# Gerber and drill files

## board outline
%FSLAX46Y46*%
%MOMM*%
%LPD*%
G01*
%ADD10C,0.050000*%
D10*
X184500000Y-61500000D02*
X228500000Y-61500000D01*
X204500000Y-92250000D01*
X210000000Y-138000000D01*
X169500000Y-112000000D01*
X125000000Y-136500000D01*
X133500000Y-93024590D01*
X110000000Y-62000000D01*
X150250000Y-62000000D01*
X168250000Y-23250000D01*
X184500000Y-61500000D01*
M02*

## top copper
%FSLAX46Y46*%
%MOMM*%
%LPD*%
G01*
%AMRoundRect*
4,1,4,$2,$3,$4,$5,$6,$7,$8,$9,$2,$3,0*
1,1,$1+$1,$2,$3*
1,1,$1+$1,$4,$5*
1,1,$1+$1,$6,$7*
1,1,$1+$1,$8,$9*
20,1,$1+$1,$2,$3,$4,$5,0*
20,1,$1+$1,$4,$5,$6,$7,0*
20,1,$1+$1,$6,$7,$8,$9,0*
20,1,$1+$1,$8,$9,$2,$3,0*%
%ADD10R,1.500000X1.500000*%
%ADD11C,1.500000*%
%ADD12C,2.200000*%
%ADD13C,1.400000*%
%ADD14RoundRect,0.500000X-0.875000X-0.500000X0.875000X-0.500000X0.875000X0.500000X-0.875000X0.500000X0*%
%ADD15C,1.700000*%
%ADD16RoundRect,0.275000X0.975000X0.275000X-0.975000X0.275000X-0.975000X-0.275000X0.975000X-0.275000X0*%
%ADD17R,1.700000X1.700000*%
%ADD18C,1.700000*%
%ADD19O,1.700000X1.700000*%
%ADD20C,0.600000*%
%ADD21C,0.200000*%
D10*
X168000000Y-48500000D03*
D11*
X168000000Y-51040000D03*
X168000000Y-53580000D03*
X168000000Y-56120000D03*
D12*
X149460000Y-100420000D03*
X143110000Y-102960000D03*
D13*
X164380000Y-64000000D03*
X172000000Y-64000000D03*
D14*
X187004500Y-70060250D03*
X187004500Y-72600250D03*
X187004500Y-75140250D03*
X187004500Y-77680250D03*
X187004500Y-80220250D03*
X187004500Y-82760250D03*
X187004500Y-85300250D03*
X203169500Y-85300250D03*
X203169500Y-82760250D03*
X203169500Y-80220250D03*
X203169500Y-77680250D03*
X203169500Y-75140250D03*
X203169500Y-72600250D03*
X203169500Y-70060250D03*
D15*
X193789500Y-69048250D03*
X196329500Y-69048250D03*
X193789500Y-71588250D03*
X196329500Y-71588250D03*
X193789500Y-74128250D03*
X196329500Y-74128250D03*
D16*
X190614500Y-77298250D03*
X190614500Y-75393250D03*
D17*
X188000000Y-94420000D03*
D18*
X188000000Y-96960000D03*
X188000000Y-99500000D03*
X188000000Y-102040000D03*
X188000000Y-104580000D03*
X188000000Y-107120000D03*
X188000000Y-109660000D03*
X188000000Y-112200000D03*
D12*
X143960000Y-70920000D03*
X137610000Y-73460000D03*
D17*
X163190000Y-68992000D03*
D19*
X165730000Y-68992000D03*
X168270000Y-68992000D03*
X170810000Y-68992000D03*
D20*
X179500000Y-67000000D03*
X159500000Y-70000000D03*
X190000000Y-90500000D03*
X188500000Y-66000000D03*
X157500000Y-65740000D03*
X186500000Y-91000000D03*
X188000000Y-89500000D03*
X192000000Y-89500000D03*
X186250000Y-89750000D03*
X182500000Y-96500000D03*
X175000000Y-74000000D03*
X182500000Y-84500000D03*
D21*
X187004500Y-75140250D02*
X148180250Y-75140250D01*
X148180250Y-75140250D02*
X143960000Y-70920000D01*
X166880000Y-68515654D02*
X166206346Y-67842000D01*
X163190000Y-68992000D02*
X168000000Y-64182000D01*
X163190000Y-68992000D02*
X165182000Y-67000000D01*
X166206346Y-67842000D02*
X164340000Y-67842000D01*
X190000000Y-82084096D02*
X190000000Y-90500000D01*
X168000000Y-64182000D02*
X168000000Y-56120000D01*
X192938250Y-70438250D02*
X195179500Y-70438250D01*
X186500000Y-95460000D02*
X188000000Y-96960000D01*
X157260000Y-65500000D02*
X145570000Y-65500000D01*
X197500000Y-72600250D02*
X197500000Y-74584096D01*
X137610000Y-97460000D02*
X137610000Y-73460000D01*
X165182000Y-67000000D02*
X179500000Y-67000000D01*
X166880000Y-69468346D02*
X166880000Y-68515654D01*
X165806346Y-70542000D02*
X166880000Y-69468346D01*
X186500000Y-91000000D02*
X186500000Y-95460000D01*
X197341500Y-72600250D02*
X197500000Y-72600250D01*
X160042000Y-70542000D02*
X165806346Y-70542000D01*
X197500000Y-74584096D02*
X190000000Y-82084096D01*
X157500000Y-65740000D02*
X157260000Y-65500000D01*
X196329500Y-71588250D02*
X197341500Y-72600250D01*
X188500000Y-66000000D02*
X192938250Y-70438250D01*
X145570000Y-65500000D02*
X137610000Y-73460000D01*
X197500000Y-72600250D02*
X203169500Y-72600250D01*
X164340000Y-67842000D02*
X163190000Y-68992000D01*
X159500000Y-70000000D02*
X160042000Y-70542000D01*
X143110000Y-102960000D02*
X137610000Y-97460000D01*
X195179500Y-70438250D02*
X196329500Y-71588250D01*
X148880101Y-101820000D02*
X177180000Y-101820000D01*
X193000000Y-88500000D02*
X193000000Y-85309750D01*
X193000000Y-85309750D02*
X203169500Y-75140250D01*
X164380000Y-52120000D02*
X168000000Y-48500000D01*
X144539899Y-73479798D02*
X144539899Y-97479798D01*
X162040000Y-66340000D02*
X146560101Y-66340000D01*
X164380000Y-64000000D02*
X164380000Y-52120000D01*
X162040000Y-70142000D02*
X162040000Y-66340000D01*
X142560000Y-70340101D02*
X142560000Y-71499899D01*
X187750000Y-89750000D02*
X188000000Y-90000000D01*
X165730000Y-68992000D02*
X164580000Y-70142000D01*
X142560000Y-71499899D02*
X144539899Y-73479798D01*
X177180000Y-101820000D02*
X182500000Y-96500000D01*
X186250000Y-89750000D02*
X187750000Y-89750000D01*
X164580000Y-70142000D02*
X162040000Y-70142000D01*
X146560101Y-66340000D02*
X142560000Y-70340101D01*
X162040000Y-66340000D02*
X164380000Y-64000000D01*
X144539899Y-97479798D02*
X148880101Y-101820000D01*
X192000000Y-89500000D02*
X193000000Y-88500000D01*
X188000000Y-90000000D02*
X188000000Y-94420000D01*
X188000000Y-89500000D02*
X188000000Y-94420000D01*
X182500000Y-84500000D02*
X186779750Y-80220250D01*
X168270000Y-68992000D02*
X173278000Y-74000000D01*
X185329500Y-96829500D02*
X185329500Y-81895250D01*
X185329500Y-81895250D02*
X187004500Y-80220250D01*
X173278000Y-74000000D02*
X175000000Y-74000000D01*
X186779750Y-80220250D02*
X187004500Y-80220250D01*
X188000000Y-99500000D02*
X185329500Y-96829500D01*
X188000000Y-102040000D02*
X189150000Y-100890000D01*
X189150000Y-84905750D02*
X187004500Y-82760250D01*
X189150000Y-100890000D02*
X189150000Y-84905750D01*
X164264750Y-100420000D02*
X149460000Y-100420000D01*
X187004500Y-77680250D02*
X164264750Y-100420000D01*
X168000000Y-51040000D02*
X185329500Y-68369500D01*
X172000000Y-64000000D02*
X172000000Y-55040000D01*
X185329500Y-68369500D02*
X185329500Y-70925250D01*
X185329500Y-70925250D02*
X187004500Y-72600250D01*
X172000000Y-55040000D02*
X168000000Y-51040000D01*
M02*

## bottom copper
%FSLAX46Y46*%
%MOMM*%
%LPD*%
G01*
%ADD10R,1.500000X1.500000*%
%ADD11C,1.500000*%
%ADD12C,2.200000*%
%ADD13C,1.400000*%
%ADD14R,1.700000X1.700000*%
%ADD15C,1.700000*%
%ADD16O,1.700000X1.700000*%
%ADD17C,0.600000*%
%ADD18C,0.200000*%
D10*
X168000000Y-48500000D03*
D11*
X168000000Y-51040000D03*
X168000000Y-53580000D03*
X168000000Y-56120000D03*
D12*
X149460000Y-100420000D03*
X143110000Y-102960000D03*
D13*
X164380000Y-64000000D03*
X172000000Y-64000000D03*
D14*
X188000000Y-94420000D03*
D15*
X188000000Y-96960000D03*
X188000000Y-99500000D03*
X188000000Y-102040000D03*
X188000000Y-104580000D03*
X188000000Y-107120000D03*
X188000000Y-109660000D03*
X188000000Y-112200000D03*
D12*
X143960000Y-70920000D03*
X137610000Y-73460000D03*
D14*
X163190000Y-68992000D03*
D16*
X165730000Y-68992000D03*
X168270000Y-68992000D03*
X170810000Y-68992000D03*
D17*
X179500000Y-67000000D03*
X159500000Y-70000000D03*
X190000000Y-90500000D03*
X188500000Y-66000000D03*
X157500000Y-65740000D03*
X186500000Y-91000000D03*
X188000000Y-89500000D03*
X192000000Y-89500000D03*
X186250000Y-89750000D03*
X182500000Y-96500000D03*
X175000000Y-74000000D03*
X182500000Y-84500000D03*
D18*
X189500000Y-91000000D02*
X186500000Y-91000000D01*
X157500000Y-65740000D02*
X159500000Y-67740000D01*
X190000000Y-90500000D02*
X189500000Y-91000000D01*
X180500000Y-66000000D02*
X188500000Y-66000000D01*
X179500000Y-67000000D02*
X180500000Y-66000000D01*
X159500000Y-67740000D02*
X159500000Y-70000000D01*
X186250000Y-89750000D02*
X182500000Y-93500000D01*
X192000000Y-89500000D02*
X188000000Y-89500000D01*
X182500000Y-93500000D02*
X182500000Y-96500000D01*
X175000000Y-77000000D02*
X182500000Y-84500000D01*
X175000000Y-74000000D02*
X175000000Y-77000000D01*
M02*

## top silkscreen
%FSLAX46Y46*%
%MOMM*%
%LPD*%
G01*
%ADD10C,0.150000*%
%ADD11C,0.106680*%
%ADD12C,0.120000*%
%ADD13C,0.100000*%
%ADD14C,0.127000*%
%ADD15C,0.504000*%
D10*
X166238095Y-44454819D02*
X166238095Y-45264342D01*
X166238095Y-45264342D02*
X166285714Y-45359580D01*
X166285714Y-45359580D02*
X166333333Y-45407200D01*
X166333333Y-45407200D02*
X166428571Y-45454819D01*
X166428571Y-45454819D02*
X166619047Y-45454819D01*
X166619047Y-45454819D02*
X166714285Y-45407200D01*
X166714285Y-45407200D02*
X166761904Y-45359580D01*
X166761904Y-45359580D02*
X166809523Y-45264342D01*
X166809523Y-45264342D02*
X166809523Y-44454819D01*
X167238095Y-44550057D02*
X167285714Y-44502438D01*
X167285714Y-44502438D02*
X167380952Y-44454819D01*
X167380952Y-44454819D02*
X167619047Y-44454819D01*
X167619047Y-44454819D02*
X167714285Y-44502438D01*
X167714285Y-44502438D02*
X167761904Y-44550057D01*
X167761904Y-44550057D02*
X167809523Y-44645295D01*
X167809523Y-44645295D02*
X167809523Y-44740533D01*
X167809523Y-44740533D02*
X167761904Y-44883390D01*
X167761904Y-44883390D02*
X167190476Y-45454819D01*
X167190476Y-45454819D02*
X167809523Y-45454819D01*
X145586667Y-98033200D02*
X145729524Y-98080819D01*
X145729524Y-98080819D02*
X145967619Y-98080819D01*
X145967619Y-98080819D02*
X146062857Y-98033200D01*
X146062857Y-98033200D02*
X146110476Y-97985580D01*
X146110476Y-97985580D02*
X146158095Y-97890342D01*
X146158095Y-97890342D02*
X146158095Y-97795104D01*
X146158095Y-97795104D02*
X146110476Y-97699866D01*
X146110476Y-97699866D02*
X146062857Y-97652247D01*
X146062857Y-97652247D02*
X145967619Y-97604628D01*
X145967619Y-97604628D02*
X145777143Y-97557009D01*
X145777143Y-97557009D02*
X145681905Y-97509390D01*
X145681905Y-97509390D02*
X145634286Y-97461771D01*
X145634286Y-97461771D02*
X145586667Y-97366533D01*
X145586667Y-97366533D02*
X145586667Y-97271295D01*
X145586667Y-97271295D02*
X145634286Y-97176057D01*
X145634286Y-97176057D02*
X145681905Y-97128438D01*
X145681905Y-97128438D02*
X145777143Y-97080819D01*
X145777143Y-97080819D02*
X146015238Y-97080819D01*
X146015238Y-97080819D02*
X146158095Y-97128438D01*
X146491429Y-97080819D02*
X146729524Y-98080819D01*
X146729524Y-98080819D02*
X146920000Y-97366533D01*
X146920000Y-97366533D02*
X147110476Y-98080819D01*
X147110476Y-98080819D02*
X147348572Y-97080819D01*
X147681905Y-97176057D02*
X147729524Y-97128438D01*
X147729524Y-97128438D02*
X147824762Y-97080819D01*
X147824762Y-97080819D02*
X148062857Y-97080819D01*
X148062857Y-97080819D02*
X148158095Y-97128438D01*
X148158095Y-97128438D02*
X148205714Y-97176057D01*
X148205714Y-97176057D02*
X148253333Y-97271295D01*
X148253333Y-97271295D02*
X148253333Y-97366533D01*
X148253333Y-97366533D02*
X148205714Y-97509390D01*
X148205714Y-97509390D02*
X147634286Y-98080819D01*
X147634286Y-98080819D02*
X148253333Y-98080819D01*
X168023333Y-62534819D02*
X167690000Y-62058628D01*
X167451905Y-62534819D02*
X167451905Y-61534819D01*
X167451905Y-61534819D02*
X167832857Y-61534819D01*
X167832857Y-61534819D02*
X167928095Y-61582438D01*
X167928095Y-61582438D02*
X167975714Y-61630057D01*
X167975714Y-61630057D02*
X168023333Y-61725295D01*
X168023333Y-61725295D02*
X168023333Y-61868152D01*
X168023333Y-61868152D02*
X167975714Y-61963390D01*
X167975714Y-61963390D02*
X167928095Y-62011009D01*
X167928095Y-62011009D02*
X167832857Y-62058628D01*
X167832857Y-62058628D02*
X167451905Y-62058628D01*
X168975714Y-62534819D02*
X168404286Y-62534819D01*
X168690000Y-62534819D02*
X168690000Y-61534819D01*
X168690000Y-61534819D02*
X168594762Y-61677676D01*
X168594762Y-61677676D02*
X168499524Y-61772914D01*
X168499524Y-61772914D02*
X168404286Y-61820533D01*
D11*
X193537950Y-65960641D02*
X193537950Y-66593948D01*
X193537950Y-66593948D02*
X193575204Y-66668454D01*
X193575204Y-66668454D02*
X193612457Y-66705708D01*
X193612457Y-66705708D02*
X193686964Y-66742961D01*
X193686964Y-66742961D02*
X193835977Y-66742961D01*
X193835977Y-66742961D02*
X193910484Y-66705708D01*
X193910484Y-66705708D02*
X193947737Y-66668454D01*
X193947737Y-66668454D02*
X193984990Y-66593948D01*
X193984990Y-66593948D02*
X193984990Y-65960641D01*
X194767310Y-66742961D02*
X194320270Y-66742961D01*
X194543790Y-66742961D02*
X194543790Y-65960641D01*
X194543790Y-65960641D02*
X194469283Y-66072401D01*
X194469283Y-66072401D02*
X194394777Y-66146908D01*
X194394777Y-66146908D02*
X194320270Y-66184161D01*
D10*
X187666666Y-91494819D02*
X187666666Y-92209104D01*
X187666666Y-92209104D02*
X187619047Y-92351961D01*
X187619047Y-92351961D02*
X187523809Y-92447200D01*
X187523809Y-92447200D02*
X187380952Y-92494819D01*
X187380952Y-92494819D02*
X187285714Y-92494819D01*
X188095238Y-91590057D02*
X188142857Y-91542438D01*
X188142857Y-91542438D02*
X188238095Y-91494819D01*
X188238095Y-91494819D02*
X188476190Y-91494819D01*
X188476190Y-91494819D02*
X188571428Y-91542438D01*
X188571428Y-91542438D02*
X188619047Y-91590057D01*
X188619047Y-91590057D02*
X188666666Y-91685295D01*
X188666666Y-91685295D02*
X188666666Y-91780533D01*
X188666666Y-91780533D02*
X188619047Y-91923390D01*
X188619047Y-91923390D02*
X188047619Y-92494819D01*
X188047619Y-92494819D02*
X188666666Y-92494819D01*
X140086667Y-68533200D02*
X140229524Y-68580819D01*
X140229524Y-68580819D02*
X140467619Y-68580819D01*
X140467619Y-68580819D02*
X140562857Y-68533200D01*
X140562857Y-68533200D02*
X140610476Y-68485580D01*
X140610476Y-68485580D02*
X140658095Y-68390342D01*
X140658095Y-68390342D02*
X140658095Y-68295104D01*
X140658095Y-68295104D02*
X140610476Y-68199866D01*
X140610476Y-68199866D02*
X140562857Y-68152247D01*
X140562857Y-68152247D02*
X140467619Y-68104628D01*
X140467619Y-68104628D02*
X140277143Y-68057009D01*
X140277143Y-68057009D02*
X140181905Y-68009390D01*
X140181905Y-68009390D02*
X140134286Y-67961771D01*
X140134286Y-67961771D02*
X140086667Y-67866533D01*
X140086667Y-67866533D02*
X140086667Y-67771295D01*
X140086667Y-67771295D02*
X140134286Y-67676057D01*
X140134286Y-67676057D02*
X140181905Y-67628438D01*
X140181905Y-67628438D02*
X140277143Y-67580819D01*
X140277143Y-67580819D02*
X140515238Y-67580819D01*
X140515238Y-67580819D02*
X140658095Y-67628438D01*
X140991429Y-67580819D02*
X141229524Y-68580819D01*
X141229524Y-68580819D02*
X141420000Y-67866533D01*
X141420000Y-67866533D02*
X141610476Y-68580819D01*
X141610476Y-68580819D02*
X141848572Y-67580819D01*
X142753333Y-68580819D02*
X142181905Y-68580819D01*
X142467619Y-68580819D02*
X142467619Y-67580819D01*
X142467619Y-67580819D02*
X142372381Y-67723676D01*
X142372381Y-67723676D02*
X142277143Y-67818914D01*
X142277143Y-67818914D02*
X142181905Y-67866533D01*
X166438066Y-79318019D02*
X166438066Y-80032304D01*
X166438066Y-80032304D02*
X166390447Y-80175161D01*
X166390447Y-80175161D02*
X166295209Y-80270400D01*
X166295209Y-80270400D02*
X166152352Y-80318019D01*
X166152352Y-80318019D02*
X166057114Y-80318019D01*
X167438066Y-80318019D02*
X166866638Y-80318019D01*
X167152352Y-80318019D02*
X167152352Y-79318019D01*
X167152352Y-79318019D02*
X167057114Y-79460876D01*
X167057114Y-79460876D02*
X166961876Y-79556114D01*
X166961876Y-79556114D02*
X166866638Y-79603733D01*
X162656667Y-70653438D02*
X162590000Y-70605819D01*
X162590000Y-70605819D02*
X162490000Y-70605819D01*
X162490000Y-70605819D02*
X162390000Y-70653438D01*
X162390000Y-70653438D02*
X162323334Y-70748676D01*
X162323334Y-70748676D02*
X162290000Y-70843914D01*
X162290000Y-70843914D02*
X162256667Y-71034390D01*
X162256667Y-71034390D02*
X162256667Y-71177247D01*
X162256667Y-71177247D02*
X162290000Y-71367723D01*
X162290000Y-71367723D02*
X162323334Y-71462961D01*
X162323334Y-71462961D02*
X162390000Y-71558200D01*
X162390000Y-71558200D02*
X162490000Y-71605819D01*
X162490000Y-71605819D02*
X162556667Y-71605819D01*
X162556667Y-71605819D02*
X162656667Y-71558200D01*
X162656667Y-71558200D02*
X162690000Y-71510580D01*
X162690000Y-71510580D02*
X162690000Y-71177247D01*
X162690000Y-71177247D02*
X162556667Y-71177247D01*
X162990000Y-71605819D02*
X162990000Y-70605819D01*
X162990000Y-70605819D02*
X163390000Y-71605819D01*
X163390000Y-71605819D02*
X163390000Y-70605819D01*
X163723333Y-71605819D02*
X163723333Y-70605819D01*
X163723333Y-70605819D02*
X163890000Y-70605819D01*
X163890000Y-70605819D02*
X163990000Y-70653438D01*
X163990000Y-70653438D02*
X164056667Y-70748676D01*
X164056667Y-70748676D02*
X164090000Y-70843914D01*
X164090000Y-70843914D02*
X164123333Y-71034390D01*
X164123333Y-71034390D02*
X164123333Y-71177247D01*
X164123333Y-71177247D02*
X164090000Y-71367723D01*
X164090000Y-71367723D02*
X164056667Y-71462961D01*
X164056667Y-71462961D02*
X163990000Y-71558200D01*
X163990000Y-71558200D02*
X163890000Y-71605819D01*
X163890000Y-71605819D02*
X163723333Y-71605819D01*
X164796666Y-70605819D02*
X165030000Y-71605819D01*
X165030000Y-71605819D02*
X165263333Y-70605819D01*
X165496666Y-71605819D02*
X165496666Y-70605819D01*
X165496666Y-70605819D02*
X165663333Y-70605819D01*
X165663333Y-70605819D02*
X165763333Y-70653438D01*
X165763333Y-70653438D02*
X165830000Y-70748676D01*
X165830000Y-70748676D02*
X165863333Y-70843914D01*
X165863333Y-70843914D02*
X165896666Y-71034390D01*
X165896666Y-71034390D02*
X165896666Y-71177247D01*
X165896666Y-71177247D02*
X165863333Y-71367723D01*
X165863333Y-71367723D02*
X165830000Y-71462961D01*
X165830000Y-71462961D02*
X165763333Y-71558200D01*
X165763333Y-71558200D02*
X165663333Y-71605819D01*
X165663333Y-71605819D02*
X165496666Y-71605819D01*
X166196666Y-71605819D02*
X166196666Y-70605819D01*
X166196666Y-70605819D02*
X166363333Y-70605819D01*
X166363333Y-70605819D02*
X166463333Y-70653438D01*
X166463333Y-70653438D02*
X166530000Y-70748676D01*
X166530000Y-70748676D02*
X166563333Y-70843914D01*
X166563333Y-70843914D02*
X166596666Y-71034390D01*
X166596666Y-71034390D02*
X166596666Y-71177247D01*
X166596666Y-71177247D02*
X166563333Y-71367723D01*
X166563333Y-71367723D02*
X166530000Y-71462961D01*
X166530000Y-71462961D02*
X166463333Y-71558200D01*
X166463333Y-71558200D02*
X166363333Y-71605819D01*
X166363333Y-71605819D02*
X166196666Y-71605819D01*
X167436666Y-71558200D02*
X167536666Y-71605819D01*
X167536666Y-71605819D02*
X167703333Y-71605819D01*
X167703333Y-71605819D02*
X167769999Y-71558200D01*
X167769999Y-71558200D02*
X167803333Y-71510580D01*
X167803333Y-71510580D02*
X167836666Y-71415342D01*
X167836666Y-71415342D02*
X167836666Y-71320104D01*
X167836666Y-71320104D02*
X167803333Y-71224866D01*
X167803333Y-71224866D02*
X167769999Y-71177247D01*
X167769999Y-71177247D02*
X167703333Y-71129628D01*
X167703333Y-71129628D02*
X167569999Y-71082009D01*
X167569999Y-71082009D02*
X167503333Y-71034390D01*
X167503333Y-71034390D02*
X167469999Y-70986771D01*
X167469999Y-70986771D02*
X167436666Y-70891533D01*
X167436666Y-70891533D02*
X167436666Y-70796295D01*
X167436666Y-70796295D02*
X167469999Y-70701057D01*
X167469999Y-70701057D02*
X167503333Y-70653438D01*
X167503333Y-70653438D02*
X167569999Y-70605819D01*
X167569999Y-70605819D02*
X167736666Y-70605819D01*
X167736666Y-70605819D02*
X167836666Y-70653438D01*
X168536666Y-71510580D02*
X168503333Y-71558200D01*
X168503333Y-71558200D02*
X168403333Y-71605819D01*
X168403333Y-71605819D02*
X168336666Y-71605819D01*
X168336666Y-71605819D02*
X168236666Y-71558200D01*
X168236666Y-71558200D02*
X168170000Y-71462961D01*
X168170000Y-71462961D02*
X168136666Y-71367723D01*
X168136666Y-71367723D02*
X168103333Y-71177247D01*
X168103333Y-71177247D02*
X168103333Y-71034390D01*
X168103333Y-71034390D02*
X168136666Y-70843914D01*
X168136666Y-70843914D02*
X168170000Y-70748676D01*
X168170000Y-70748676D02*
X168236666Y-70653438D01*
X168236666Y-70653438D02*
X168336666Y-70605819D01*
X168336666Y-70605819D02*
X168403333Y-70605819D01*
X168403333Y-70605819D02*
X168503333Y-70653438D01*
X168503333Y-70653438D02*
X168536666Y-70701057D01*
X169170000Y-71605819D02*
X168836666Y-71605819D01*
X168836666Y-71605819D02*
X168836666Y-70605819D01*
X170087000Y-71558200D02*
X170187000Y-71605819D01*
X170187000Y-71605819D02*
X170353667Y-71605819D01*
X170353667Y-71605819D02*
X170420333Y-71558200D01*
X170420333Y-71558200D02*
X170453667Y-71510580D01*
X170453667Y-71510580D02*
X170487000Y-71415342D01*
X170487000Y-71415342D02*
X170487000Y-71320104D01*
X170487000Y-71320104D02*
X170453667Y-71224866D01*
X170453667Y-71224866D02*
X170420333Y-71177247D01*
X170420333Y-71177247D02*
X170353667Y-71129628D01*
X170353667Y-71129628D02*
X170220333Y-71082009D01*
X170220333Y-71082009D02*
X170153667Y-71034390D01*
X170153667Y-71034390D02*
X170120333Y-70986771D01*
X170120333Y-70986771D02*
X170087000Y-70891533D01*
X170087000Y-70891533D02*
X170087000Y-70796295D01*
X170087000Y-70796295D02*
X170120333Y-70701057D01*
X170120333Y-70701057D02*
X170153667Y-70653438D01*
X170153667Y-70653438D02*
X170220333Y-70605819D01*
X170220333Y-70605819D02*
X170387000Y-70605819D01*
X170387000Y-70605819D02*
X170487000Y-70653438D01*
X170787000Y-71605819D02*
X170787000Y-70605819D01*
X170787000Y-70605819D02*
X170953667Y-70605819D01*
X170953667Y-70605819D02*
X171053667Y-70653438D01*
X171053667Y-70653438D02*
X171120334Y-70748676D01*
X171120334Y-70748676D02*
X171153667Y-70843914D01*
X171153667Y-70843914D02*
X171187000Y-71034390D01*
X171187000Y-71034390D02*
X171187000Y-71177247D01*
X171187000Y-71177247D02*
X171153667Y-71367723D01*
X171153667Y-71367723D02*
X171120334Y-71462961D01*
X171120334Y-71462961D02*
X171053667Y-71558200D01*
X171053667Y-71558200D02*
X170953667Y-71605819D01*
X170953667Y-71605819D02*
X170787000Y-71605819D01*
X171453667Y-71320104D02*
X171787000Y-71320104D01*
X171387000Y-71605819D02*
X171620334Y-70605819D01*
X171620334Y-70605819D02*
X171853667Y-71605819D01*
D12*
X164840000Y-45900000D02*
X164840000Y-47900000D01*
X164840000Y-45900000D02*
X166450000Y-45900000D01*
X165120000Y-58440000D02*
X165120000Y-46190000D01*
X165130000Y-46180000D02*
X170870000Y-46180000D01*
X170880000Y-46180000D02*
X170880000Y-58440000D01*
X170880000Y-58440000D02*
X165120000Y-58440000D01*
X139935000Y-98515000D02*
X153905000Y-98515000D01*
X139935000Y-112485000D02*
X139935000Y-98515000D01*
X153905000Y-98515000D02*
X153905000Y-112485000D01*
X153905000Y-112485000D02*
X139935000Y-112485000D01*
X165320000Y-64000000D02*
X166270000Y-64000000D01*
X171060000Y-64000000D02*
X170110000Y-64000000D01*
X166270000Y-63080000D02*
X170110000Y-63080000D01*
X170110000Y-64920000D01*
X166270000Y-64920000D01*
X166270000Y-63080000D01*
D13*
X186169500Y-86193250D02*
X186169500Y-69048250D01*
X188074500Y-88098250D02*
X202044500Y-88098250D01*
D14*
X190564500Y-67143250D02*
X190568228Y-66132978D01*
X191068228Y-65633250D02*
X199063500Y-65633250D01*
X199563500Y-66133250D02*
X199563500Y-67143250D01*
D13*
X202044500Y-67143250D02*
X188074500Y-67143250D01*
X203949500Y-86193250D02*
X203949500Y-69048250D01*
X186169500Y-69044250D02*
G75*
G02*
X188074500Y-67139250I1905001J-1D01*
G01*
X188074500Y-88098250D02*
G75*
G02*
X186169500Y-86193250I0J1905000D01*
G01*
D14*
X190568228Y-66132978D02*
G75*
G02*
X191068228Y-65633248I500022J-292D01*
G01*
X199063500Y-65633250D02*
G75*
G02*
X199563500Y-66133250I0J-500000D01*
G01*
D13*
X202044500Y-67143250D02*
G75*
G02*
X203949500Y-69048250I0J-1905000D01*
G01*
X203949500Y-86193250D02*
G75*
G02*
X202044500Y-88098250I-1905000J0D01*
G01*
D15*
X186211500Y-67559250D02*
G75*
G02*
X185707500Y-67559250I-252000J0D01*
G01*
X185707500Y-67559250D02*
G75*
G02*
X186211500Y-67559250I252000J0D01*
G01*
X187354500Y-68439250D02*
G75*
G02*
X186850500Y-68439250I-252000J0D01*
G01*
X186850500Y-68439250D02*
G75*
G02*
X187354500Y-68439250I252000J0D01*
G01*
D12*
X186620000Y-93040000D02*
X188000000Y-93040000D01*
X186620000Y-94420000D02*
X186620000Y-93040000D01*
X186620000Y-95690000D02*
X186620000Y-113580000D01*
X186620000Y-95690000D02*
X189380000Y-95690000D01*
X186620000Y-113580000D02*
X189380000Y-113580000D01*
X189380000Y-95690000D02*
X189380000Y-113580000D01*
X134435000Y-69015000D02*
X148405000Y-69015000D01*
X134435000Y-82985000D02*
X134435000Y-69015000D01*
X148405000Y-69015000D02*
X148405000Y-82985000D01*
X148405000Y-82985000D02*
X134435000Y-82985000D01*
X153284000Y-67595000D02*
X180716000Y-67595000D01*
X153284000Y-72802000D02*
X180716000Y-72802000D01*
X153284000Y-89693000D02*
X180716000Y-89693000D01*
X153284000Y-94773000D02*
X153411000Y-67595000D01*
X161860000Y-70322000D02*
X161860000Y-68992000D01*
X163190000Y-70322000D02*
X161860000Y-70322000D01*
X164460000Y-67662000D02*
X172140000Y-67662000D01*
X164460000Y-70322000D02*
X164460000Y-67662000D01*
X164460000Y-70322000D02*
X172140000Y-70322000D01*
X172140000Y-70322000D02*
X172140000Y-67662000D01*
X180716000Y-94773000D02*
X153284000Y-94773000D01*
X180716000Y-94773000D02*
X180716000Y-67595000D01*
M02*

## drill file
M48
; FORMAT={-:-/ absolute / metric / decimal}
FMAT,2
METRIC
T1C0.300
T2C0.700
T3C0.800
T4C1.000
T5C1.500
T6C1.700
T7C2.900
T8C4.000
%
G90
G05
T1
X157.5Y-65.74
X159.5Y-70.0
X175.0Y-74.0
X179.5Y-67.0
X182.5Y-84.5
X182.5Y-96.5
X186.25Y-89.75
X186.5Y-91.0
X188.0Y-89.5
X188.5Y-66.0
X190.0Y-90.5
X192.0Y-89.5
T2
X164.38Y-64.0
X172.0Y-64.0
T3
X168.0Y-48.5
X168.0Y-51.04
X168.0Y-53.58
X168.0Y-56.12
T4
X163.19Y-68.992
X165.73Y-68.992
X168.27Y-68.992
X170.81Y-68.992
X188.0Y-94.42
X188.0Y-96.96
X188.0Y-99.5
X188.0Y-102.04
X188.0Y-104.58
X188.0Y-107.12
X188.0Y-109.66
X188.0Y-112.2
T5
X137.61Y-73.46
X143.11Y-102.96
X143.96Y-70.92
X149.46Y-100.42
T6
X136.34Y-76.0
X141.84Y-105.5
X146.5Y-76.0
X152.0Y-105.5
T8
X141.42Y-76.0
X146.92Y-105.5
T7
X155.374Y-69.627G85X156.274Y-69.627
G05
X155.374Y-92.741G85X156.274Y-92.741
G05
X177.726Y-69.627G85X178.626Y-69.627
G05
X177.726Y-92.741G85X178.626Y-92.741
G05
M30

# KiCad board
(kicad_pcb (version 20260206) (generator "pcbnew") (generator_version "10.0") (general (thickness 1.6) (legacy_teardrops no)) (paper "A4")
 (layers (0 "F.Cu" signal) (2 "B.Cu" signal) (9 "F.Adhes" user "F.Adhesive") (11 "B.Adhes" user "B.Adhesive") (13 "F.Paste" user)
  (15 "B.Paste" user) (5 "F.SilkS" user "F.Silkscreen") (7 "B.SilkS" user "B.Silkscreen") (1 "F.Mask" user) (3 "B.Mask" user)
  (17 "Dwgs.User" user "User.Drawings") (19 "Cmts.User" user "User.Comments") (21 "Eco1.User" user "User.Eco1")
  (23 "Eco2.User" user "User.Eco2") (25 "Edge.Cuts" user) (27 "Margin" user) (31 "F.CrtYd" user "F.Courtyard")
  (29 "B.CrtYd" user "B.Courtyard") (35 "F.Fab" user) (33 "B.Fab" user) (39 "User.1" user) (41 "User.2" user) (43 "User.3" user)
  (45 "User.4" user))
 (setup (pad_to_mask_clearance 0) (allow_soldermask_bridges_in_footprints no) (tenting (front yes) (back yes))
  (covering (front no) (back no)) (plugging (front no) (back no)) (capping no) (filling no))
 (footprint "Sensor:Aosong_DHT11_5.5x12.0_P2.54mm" (layer "F.Cu") (at 168 48.5)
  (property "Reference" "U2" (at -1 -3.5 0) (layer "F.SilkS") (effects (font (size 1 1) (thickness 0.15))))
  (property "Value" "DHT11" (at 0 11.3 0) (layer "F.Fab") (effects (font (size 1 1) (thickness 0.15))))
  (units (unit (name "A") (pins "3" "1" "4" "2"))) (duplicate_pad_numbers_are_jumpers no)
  (fp_line (start -3.16 -2.6) (end -3.16 -0.6) (stroke (width 0.12) (type solid)) (layer "F.SilkS"))
  (fp_line (start -3.16 -2.6) (end -1.55 -2.6) (stroke (width 0.12) (type solid)) (layer "F.SilkS"))
  (fp_line (start -2.88 9.94) (end -2.88 -2.31) (stroke (width 0.12) (type solid)) (layer "F.SilkS"))
  (fp_line (start -2.87 -2.32) (end 2.87 -2.32) (stroke (width 0.12) (type solid)) (layer "F.SilkS"))
  (fp_line (start 2.88 -2.32) (end 2.88 9.94) (stroke (width 0.12) (type solid)) (layer "F.SilkS"))
  (fp_line (start 2.88 9.94) (end -2.88 9.94) (stroke (width 0.12) (type solid)) (layer "F.SilkS"))
  (pad "1" thru_hole rect (at 0 0) (size 1.5 1.5) (drill 0.8) (layers "*.Cu" "*.Mask") (remove_unused_layers no) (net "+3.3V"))
  (pad "2" thru_hole circle (at 0 2.54) (size 1.5 1.5) (drill 0.8) (layers "*.Cu" "*.Mask") (remove_unused_layers no) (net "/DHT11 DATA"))
  (pad "3" thru_hole circle (at 0 5.08) (size 1.5 1.5) (drill 0.8) (layers "*.Cu" "*.Mask") (remove_unused_layers no)
   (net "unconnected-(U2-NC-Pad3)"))
  (pad "4" thru_hole circle (at 0 7.62) (size 1.5 1.5) (drill 0.8) (layers "*.Cu" "*.Mask") (remove_unused_layers no) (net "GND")))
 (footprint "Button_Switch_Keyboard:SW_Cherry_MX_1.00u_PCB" (layer "F.Cu") (at 149.46 100.42)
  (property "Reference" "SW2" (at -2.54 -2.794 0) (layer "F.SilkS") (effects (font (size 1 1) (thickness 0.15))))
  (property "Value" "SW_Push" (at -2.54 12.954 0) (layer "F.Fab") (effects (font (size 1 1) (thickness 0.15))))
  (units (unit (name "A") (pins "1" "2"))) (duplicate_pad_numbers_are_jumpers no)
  (fp_line (start -9.525 -1.905) (end 4.445 -1.905) (stroke (width 0.12) (type solid)) (layer "F.SilkS"))
  (fp_line (start -9.525 12.065) (end -9.525 -1.905) (stroke (width 0.12) (type solid)) (layer "F.SilkS"))
  (fp_line (start 4.445 -1.905) (end 4.445 12.065) (stroke (width 0.12) (type solid)) (layer "F.SilkS"))
  (fp_line (start 4.445 12.065) (end -9.525 12.065) (stroke (width 0.12) (type solid)) (layer "F.SilkS"))
  (pad "" np_thru_hole circle (at -7.62 5.08) (size 1.7 1.7) (drill 1.7) (layers "*.Cu" "*.Mask"))
  (pad "" np_thru_hole circle (at -2.54 5.08) (size 4 4) (drill 4) (layers "*.Cu" "*.Mask"))
  (pad "" np_thru_hole circle (at 2.54 5.08) (size 1.7 1.7) (drill 1.7) (layers "*.Cu" "*.Mask"))
  (pad "1" thru_hole circle (at 0 0) (size 2.2 2.2) (drill 1.5) (layers "*.Cu" "*.Mask") (remove_unused_layers no) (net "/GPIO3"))
  (pad "2" thru_hole circle (at -6.35 2.54) (size 2.2 2.2) (drill 1.5) (layers "*.Cu" "*.Mask") (remove_unused_layers no) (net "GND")))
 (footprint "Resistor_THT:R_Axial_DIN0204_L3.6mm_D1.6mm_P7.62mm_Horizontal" (layer "F.Cu") (at 164.38 64)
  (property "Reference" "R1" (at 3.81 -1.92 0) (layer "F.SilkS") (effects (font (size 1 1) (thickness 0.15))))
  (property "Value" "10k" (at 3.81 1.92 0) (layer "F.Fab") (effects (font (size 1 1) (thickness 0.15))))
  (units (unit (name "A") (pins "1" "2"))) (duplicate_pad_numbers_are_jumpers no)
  (fp_line (start 0.94 0) (end 1.89 0) (stroke (width 0.12) (type solid)) (layer "F.SilkS"))
  (fp_line (start 6.68 0) (end 5.73 0) (stroke (width 0.12) (type solid)) (layer "F.SilkS"))
  (fp_rect (start 1.89 -0.92) (end 5.73 0.92) (stroke (width 0.12) (type solid)) (fill no) (layer "F.SilkS"))
  (pad "1" thru_hole circle (at 0 0) (size 1.4 1.4) (drill 0.7) (layers "*.Cu" "*.Mask") (remove_unused_layers no) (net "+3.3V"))
  (pad "2" thru_hole circle (at 7.62 0) (size 1.4 1.4) (drill 0.7) (layers "*.Cu" "*.Mask") (remove_unused_layers no) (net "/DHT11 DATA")))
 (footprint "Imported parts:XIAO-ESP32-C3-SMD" (layer "F.Cu") (at 186.1695 88.18025)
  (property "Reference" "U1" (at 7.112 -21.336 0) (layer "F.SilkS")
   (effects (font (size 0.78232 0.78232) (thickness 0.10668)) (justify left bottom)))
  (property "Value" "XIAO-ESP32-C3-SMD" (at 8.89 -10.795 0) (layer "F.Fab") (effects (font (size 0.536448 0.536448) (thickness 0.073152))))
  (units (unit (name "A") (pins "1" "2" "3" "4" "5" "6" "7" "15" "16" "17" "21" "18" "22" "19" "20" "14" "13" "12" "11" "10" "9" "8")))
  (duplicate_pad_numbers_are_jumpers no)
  (fp_line (start 0 -1.987) (end 0 -19.132) (stroke (width 0.1) (type solid)) (layer "F.SilkS"))
  (fp_line (start 1.905 -0.082) (end 15.875 -0.082) (stroke (width 0.1) (type solid)) (layer "F.SilkS"))
  (fp_line (start 4.395 -21.037) (end 4.398728 -22.047272) (stroke (width 0.127) (type solid)) (layer "F.SilkS"))
  (fp_line (start 4.898728 -22.547) (end 12.894 -22.547) (stroke (width 0.127) (type solid)) (layer "F.SilkS"))
  (fp_line (start 13.394 -22.047) (end 13.394 -21.037) (stroke (width 0.127) (type solid)) (layer "F.SilkS"))
  (fp_line (start 15.875 -21.037) (end 1.905 -21.037) (stroke (width 0.1) (type solid)) (layer "F.SilkS"))
  (fp_line (start 17.78 -1.987) (end 17.78 -19.132) (stroke (width 0.1) (type solid)) (layer "F.SilkS"))
  (fp_arc (start 0 -19.136) (mid 0.557962 -20.483038) (end 1.905 -21.041) (stroke (width 0.1) (type solid)) (layer "F.SilkS"))
  (fp_arc (start 1.905 -0.082) (mid 0.557962 -0.639962) (end 0 -1.987) (stroke (width 0.1) (type solid)) (layer "F.SilkS"))
  (fp_arc (start 4.398728 -22.047272) (mid 4.545272 -22.40064) (end 4.898728 -22.547) (stroke (width 0.127) (type default))
   (layer "F.SilkS"))
  (fp_arc (start 12.894 -22.547) (mid 13.247553 -22.400553) (end 13.394 -22.047) (stroke (width 0.127) (type default)) (layer "F.SilkS"))
  (fp_arc (start 15.875 -21.037) (mid 17.222038 -20.479038) (end 17.78 -19.132) (stroke (width 0.1) (type solid)) (layer "F.SilkS"))
  (fp_arc (start 17.78 -1.987) (mid 17.222038 -0.639962) (end 15.875 -0.082) (stroke (width 0.1) (type solid)) (layer "F.SilkS"))
  (fp_circle (center -0.21 -20.621) (end -0.21 -20.875) (stroke (width 0.5) (type solid)) (fill yes) (layer "F.SilkS"))
  (fp_circle (center 0.933 -19.741) (end 0.933 -19.995) (stroke (width 0.5) (type solid)) (fill yes) (layer "F.SilkS"))
  (pad "1" smd roundrect (at 0.835 -18.12) (size 2.75 2) (layers "F.Cu" "F.Mask" "F.Paste") (roundrect_rratio 0.25)
   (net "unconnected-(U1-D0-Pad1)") (solder_mask_margin 0.0508) (thermal_bridge_angle 45))
  (pad "2" smd roundrect (at 0.835 -15.58) (size 2.75 2) (layers "F.Cu" "F.Mask" "F.Paste") (roundrect_rratio 0.25) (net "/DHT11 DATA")
   (solder_mask_margin 0.0508) (thermal_bridge_angle 45))
  (pad "3" smd roundrect (at 0.835 -13.04) (size 2.75 2) (layers "F.Cu" "F.Mask" "F.Paste") (roundrect_rratio 0.25) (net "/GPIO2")
   (solder_mask_margin 0.0508) (thermal_bridge_angle 45))
  (pad "4" smd roundrect (at 0.835 -10.5) (size 2.75 2) (layers "F.Cu" "F.Mask" "F.Paste") (roundrect_rratio 0.25) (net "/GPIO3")
   (solder_mask_margin 0.0508) (thermal_bridge_angle 45))
  (pad "5" smd roundrect (at 0.835 -7.96) (size 2.75 2) (layers "F.Cu" "F.Mask" "F.Paste") (roundrect_rratio 0.25) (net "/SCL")
   (solder_mask_margin 0.0508) (thermal_bridge_angle 45))
  (pad "6" smd roundrect (at 0.835 -5.42) (size 2.75 2) (layers "F.Cu" "F.Mask" "F.Paste") (roundrect_rratio 0.25) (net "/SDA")
   (solder_mask_margin 0.0508) (thermal_bridge_angle 45))
  (pad "7" smd roundrect (at 0.835 -2.88) (size 2.75 2) (layers "F.Cu" "F.Mask" "F.Paste") (roundrect_rratio 0.25)
   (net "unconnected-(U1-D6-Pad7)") (solder_mask_margin 0.0508) (thermal_bridge_angle 45))
  (pad "8" smd roundrect (at 17 -2.88) (size 2.75 2) (layers "F.Cu" "F.Mask" "F.Paste") (roundrect_rratio 0.25)
   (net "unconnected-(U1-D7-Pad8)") (solder_mask_margin 0.0508) (thermal_bridge_angle 45))
  (pad "9" smd roundrect (at 17 -5.42) (size 2.75 2) (layers "F.Cu" "F.Mask" "F.Paste") (roundrect_rratio 0.25)
   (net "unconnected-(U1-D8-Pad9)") (solder_mask_margin 0.0508) (thermal_bridge_angle 45))
  (pad "10" smd roundrect (at 17 -7.96) (size 2.75 2) (layers "F.Cu" "F.Mask" "F.Paste") (roundrect_rratio 0.25)
   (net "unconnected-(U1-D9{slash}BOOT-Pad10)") (solder_mask_margin 0.0508) (thermal_bridge_angle 45))
  (pad "11" smd roundrect (at 17 -10.5) (size 2.75 2) (layers "F.Cu" "F.Mask" "F.Paste") (roundrect_rratio 0.25)
   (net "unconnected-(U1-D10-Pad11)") (solder_mask_margin 0.0508) (thermal_bridge_angle 45))
  (pad "12" smd roundrect (at 17 -13.04) (size 2.75 2) (layers "F.Cu" "F.Mask" "F.Paste") (roundrect_rratio 0.25) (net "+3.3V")
   (solder_mask_margin 0.0508) (thermal_bridge_angle 45))
  (pad "13" smd roundrect (at 17 -15.58) (size 2.75 2) (layers "F.Cu" "F.Mask" "F.Paste") (roundrect_rratio 0.25) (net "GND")
   (solder_mask_margin 0.0508) (thermal_bridge_angle 45))
  (pad "14" smd roundrect (at 17 -18.12) (size 2.75 2) (layers "F.Cu" "F.Mask" "F.Paste") (roundrect_rratio 0.25) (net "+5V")
   (solder_mask_margin 0.0508) (thermal_bridge_angle 45))
  (pad "15" smd circle (at 7.62 -19.132) (size 1.7 1.7) (layers "F.Cu" "F.Mask" "F.Paste") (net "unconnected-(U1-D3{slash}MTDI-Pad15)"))
  (pad "16" smd circle (at 10.16 -19.132) (size 1.7 1.7) (layers "F.Cu" "F.Mask" "F.Paste") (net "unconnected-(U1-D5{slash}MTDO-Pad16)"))
  (pad "17" smd circle (at 7.62 -16.592) (size 1.7 1.7) (layers "F.Cu" "F.Mask" "F.Paste") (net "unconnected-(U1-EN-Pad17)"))
  (pad "18" smd circle (at 10.16 -16.592) (size 1.7 1.7) (layers "F.Cu" "F.Mask" "F.Paste") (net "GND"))
  (pad "19" smd circle (at 7.62 -14.052) (size 1.7 1.7) (layers "F.Cu" "F.Mask" "F.Paste") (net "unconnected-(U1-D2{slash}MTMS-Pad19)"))
  (pad "20" smd circle (at 10.16 -14.052) (size 1.7 1.7) (layers "F.Cu" "F.Mask" "F.Paste") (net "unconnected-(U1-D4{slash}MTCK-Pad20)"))
  (pad "21" smd roundrect (at 4.445 -10.882 180) (size 2.5 1.1) (layers "F.Cu" "F.Mask" "F.Paste") (roundrect_rratio 0.25)
   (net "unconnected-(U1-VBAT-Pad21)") (thermal_bridge_angle 45))
  (pad "22" smd roundrect (at 4.445 -12.787 180) (size 2.5 1.1) (layers "F.Cu" "F.Mask" "F.Paste") (roundrect_rratio 0.25)
   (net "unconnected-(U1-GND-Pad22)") (thermal_bridge_angle 45)))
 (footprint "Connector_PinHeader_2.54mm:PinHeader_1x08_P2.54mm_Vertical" (layer "F.Cu") (at 188 94.42)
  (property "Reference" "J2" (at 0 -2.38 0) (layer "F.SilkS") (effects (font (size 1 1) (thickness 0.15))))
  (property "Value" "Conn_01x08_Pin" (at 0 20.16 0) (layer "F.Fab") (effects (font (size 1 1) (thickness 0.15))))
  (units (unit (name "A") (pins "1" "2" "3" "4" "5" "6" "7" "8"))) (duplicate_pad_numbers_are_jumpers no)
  (fp_line (start -1.38 -1.38) (end 0 -1.38) (stroke (width 0.12) (type solid)) (layer "F.SilkS"))
  (fp_line (start -1.38 0) (end -1.38 -1.38) (stroke (width 0.12) (type solid)) (layer "F.SilkS"))
  (fp_line (start -1.38 1.27) (end -1.38 19.16) (stroke (width 0.12) (type solid)) (layer "F.SilkS"))
  (fp_line (start -1.38 1.27) (end 1.38 1.27) (stroke (width 0.12) (type solid)) (layer "F.SilkS"))
  (fp_line (start -1.38 19.16) (end 1.38 19.16) (stroke (width 0.12) (type solid)) (layer "F.SilkS"))
  (fp_line (start 1.38 1.27) (end 1.38 19.16) (stroke (width 0.12) (type solid)) (layer "F.SilkS"))
  (pad "1" thru_hole rect (at 0 0) (size 1.7 1.7) (drill 1) (layers "*.Cu" "*.Mask") (remove_unused_layers no) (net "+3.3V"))
  (pad "2" thru_hole circle (at 0 2.54) (size 1.7 1.7) (drill 1) (layers "*.Cu" "*.Mask") (remove_unused_layers no) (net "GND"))
  (pad "3" thru_hole circle (at 0 5.08) (size 1.7 1.7) (drill 1) (layers "*.Cu" "*.Mask") (remove_unused_layers no) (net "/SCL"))
  (pad "4" thru_hole circle (at 0 7.62) (size 1.7 1.7) (drill 1) (layers "*.Cu" "*.Mask") (remove_unused_layers no) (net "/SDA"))
  (pad "5" thru_hole circle (at 0 10.16) (size 1.7 1.7) (drill 1) (layers "*.Cu" "*.Mask") (remove_unused_layers no)
   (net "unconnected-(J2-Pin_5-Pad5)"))
  (pad "6" thru_hole circle (at 0 12.7) (size 1.7 1.7) (drill 1) (layers "*.Cu" "*.Mask") (remove_unused_layers no)
   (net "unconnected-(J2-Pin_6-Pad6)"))
  (pad "7" thru_hole circle (at 0 15.24) (size 1.7 1.7) (drill 1) (layers "*.Cu" "*.Mask") (remove_unused_layers no)
   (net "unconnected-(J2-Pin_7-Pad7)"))
  (pad "8" thru_hole circle (at 0 17.78) (size 1.7 1.7) (drill 1) (layers "*.Cu" "*.Mask") (remove_unused_layers no)
   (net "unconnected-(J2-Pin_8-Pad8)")))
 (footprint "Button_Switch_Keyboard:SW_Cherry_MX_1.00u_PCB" (layer "F.Cu") (at 143.96 70.92)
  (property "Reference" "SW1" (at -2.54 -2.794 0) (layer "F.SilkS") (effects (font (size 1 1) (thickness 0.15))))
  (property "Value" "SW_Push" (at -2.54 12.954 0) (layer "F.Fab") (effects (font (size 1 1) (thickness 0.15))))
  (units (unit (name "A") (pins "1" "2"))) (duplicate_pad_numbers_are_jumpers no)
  (fp_line (start -9.525 -1.905) (end 4.445 -1.905) (stroke (width 0.12) (type solid)) (layer "F.SilkS"))
  (fp_line (start -9.525 12.065) (end -9.525 -1.905) (stroke (width 0.12) (type solid)) (layer "F.SilkS"))
  (fp_line (start 4.445 -1.905) (end 4.445 12.065) (stroke (width 0.12) (type solid)) (layer "F.SilkS"))
  (fp_line (start 4.445 12.065) (end -9.525 12.065) (stroke (width 0.12) (type solid)) (layer "F.SilkS"))
  (pad "" np_thru_hole circle (at -7.62 5.08) (size 1.7 1.7) (drill 1.7) (layers "*.Cu" "*.Mask"))
  (pad "" np_thru_hole circle (at -2.54 5.08) (size 4 4) (drill 4) (layers "*.Cu" "*.Mask"))
  (pad "" np_thru_hole circle (at 2.54 5.08) (size 1.7 1.7) (drill 1.7) (layers "*.Cu" "*.Mask"))
  (pad "1" thru_hole circle (at 0 0) (size 2.2 2.2) (drill 1.5) (layers "*.Cu" "*.Mask") (remove_unused_layers no) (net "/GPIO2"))
  (pad "2" thru_hole circle (at -6.35 2.54) (size 2.2 2.2) (drill 1.5) (layers "*.Cu" "*.Mask") (remove_unused_layers no) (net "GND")))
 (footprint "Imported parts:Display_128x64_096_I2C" (layer "F.Cu") (at 167 68.992)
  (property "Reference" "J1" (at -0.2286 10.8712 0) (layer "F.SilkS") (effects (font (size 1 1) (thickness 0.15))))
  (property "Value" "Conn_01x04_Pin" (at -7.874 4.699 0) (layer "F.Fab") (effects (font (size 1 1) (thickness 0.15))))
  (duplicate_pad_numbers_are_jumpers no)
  (fp_line (start -13.716 -1.397) (end 13.716 -1.397) (stroke (width 0.12) (type solid)) (layer "F.SilkS"))
  (fp_line (start -13.716 3.81) (end 13.716 3.81) (stroke (width 0.12) (type solid)) (layer "F.SilkS"))
  (fp_line (start -13.716 20.701) (end 13.716 20.701) (stroke (width 0.12) (type solid)) (layer "F.SilkS"))
  (fp_line (start -13.716 25.781) (end -13.589 -1.397) (stroke (width 0.12) (type solid)) (layer "F.SilkS"))
  (fp_line (start -5.14 1.33) (end -5.14 0) (stroke (width 0.12) (type solid)) (layer "F.SilkS"))
  (fp_line (start -3.81 1.33) (end -5.14 1.33) (stroke (width 0.12) (type solid)) (layer "F.SilkS"))
  (fp_line (start -2.54 -1.33) (end 5.14 -1.33) (stroke (width 0.12) (type solid)) (layer "F.SilkS"))
  (fp_line (start -2.54 1.33) (end -2.54 -1.33) (stroke (width 0.12) (type solid)) (layer "F.SilkS"))
  (fp_line (start -2.54 1.33) (end 5.14 1.33) (stroke (width 0.12) (type solid)) (layer "F.SilkS"))
  (fp_line (start 5.14 1.33) (end 5.14 -1.33) (stroke (width 0.12) (type solid)) (layer "F.SilkS"))
  (fp_line (start 13.716 25.781) (end -13.716 25.781) (stroke (width 0.12) (type solid)) (layer "F.SilkS"))
  (fp_line (start 13.716 25.781) (end 13.716 -1.397) (stroke (width 0.12) (type solid)) (layer "F.SilkS"))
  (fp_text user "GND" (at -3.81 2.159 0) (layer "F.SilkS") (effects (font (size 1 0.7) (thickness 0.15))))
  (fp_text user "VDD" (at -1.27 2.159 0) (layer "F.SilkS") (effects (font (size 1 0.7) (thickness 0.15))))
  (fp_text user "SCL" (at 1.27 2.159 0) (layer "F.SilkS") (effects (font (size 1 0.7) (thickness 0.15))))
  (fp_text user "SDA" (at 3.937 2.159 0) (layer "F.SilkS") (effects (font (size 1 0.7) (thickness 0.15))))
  (pad "" np_thru_hole oval (at -11.176 0.635) (size 3.8 2.9) (drill oval 3.8 2.9) (layers "*.Cu" "*.Mask"))
  (pad "" np_thru_hole oval (at -11.176 23.749) (size 3.8 2.9) (drill oval 3.8 2.9) (layers "*.Cu" "*.Mask"))
  (pad "" np_thru_hole oval (at 11.176 0.635) (size 3.8 2.9) (drill oval 3.8 2.9) (layers "*.Cu" "*.Mask"))
  (pad "" np_thru_hole oval (at 11.176 23.749) (size 3.8 2.9) (drill oval 3.8 2.9) (layers "*.Cu" "*.Mask"))
  (pad "1" thru_hole rect (at -3.81 0 90) (size 1.7 1.7) (drill 1) (layers "*.Cu" "*.Mask") (remove_unused_layers no) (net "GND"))
  (pad "2" thru_hole oval (at -1.27 0 90) (size 1.7 1.7) (drill 1) (layers "*.Cu" "*.Mask") (remove_unused_layers no) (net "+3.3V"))
  (pad "3" thru_hole oval (at 1.27 0 90) (size 1.7 1.7) (drill 1) (layers "*.Cu" "*.Mask") (remove_unused_layers no) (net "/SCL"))
  (pad "4" thru_hole oval (at 3.81 0 90) (size 1.7 1.7) (drill 1) (layers "*.Cu" "*.Mask") (remove_unused_layers no) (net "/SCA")))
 (gr_poly
  (pts (xy 184.5 61.5) (xy 228.5 61.5) (xy 204.5 92.25) (xy 210 138) (xy 169.5 112) (xy 125 136.5) (xy 133.5 93.02459) (xy 110 62)
   (xy 150.25 62) (xy 168.25 23.25))
  (stroke (width 0.05) (type solid)) (fill no) (layer "Edge.Cuts"))
 (segment (start 187.0045 75.14025) (end 148.18025 75.14025) (width 0.2) (layer "F.Cu") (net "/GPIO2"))
 (segment (start 148.18025 75.14025) (end 143.96 70.92) (width 0.2) (layer "F.Cu") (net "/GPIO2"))
 (segment (start 166.88 68.515654) (end 166.206346 67.842) (width 0.2) (layer "F.Cu") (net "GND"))
 (segment (start 163.19 68.992) (end 168 64.182) (width 0.2) (layer "F.Cu") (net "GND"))
 (segment (start 163.19 68.992) (end 165.182 67) (width 0.2) (layer "F.Cu") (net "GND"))
 (segment (start 166.206346 67.842) (end 164.34 67.842) (width 0.2) (layer "F.Cu") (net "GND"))
 (segment (start 190 82.084096) (end 190 90.5) (width 0.2) (layer "F.Cu") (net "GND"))
 (segment (start 168 64.182) (end 168 56.12) (width 0.2) (layer "F.Cu") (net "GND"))
 (segment (start 192.93825 70.43825) (end 195.1795 70.43825) (width 0.2) (layer "F.Cu") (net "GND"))
 (segment (start 186.5 95.46) (end 188 96.96) (width 0.2) (layer "F.Cu") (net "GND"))
 (segment (start 157.26 65.5) (end 145.57 65.5) (width 0.2) (layer "F.Cu") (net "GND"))
 (segment (start 197.5 72.60025) (end 197.5 74.584096) (width 0.2) (layer "F.Cu") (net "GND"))
 (segment (start 137.61 97.46) (end 137.61 73.46) (width 0.2) (layer "F.Cu") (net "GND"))
 (segment (start 165.182 67) (end 179.5 67) (width 0.2) (layer "F.Cu") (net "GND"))
 (segment (start 166.88 69.468346) (end 166.88 68.515654) (width 0.2) (layer "F.Cu") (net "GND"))
 (segment (start 165.806346 70.542) (end 166.88 69.468346) (width 0.2) (layer "F.Cu") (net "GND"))
 (segment (start 186.5 91) (end 186.5 95.46) (width 0.2) (layer "F.Cu") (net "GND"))
 (segment (start 197.3415 72.60025) (end 197.5 72.60025) (width 0.2) (layer "F.Cu") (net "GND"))
 (segment (start 160.042 70.542) (end 165.806346 70.542) (width 0.2) (layer "F.Cu") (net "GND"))
 (segment (start 197.5 74.584096) (end 190 82.084096) (width 0.2) (layer "F.Cu") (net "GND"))
 (segment (start 157.5 65.74) (end 157.26 65.5) (width 0.2) (layer "F.Cu") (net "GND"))
 (segment (start 196.3295 71.58825) (end 197.3415 72.60025) (width 0.2) (layer "F.Cu") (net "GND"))
 (segment (start 188.5 66) (end 192.93825 70.43825) (width 0.2) (layer "F.Cu") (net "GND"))
 (segment (start 145.57 65.5) (end 137.61 73.46) (width 0.2) (layer "F.Cu") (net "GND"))
 (segment (start 197.5 72.60025) (end 203.1695 72.60025) (width 0.2) (layer "F.Cu") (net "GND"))
 (segment (start 164.34 67.842) (end 163.19 68.992) (width 0.2) (layer "F.Cu") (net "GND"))
 (segment (start 159.5 70) (end 160.042 70.542) (width 0.2) (layer "F.Cu") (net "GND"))
 (segment (start 143.11 102.96) (end 137.61 97.46) (width 0.2) (layer "F.Cu") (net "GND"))
 (segment (start 195.1795 70.43825) (end 196.3295 71.58825) (width 0.2) (layer "F.Cu") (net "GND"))
 (via (at 179.5 67) (size 0.6) (drill 0.3) (layers "F.Cu" "B.Cu") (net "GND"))
 (via (at 159.5 70) (size 0.6) (drill 0.3) (layers "F.Cu" "B.Cu") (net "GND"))
 (via (at 190 90.5) (size 0.6) (drill 0.3) (layers "F.Cu" "B.Cu") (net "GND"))
 (via (at 188.5 66) (size 0.6) (drill 0.3) (layers "F.Cu" "B.Cu") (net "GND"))
 (via (at 157.5 65.74) (size 0.6) (drill 0.3) (layers "F.Cu" "B.Cu") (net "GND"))
 (via (at 186.5 91) (size 0.6) (drill 0.3) (layers "F.Cu" "B.Cu") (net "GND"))
 (segment (start 189.5 91) (end 186.5 91) (width 0.2) (layer "B.Cu") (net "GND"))
 (segment (start 157.5 65.74) (end 159.5 67.74) (width 0.2) (layer "B.Cu") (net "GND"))
 (segment (start 190 90.5) (end 189.5 91) (width 0.2) (layer "B.Cu") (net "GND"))
 (segment (start 180.5 66) (end 188.5 66) (width 0.2) (layer "B.Cu") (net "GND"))
 (segment (start 179.5 67) (end 180.5 66) (width 0.2) (layer "B.Cu") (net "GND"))
 (segment (start 159.5 67.74) (end 159.5 70) (width 0.2) (layer "B.Cu") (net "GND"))
 (segment (start 148.880101 101.82) (end 177.18 101.82) (width 0.2) (layer "F.Cu") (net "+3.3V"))
 (segment (start 193 88.5) (end 193 85.30975) (width 0.2) (layer "F.Cu") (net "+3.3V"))
 (segment (start 193 85.30975) (end 203.1695 75.14025) (width 0.2) (layer "F.Cu") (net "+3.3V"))
 (segment (start 164.38 52.12) (end 168 48.5) (width 0.2) (layer "F.Cu") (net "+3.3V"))
 (segment (start 144.539899 73.479798) (end 144.539899 97.479798) (width 0.2) (layer "F.Cu") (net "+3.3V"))
 (segment (start 162.04 66.34) (end 146.560101 66.34) (width 0.2) (layer "F.Cu") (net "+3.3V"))
 (segment (start 164.38 64) (end 164.38 52.12) (width 0.2) (layer "F.Cu") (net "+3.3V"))
 (segment (start 162.04 70.142) (end 162.04 66.34) (width 0.2) (layer "F.Cu") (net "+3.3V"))
 (segment (start 142.56 70.340101) (end 142.56 71.499899) (width 0.2) (layer "F.Cu") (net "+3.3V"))
 (segment (start 187.75 89.75) (end 188 90) (width 0.2) (layer "F.Cu") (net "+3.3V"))
 (segment (start 165.73 68.992) (end 164.58 70.142) (width 0.2) (layer "F.Cu") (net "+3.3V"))
 (segment (start 142.56 71.499899) (end 144.539899 73.479798) (width 0.2) (layer "F.Cu") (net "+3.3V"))
 (segment (start 177.18 101.82) (end 182.5 96.5) (width 0.2) (layer "F.Cu") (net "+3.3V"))
 (segment (start 186.25 89.75) (end 187.75 89.75) (width 0.2) (layer "F.Cu") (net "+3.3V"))
 (segment (start 164.58 70.142) (end 162.04 70.142) (width 0.2) (layer "F.Cu") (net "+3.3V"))
 (segment (start 146.560101 66.34) (end 142.56 70.340101) (width 0.2) (layer "F.Cu") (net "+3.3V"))
 (segment (start 162.04 66.34) (end 164.38 64) (width 0.2) (layer "F.Cu") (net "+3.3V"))
 (segment (start 144.539899 97.479798) (end 148.880101 101.82) (width 0.2) (layer "F.Cu") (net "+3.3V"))
 (segment (start 192 89.5) (end 193 88.5) (width 0.2) (layer "F.Cu") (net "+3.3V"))
 (segment (start 188 90) (end 188 94.42) (width 0.2) (layer "F.Cu") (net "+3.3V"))
 (segment (start 188 89.5) (end 188 94.42) (width 0.2) (layer "F.Cu") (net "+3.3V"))
 (via (at 188 89.5) (size 0.6) (drill 0.3) (layers "F.Cu" "B.Cu") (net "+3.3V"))
 (via (at 192 89.5) (size 0.6) (drill 0.3) (layers "F.Cu" "B.Cu") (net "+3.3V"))
 (via (at 186.25 89.75) (size 0.6) (drill 0.3) (layers "F.Cu" "B.Cu") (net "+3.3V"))
 (via (at 182.5 96.5) (size 0.6) (drill 0.3) (layers "F.Cu" "B.Cu") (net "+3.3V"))
 (segment (start 186.25 89.75) (end 182.5 93.5) (width 0.2) (layer "B.Cu") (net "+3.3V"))
 (segment (start 192 89.5) (end 188 89.5) (width 0.2) (layer "B.Cu") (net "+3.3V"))
 (segment (start 182.5 93.5) (end 182.5 96.5) (width 0.2) (layer "B.Cu") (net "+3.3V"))
 (segment (start 182.5 84.5) (end 186.77975 80.22025) (width 0.2) (layer "F.Cu") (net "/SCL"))
 (segment (start 168.27 68.992) (end 173.278 74) (width 0.2) (layer "F.Cu") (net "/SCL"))
 (segment (start 185.3295 96.8295) (end 185.3295 81.89525) (width 0.2) (layer "F.Cu") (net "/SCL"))
 (segment (start 185.3295 81.89525) (end 187.0045 80.22025) (width 0.2) (layer "F.Cu") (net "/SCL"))
 (segment (start 173.278 74) (end 175 74) (width 0.2) (layer "F.Cu") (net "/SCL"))
 (segment (start 186.77975 80.22025) (end 187.0045 80.22025) (width 0.2) (layer "F.Cu") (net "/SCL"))
 (segment (start 188 99.5) (end 185.3295 96.8295) (width 0.2) (layer "F.Cu") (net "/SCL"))
 (via (at 175 74) (size 0.6) (drill 0.3) (layers "F.Cu" "B.Cu") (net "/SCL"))
 (via (at 182.5 84.5) (size 0.6) (drill 0.3) (layers "F.Cu" "B.Cu") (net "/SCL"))
 (segment (start 175 77) (end 182.5 84.5) (width 0.2) (layer "B.Cu") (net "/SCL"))
 (segment (start 175 74) (end 175 77) (width 0.2) (layer "B.Cu") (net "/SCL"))
 (segment (start 188 102.04) (end 189.15 100.89) (width 0.2) (layer "F.Cu") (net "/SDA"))
 (segment (start 189.15 84.90575) (end 187.0045 82.76025) (width 0.2) (layer "F.Cu") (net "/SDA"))
 (segment (start 189.15 100.89) (end 189.15 84.90575) (width 0.2) (layer "F.Cu") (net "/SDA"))
 (segment (start 164.26475 100.42) (end 149.46 100.42) (width 0.2) (layer "F.Cu") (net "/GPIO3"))
 (segment (start 187.0045 77.68025) (end 164.26475 100.42) (width 0.2) (layer "F.Cu") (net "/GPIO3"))
 (segment (start 168 51.04) (end 185.3295 68.3695) (width 0.2) (layer "F.Cu") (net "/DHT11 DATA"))
 (segment (start 172 64) (end 172 55.04) (width 0.2) (layer "F.Cu") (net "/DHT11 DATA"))
 (segment (start 185.3295 68.3695) (end 185.3295 70.92525) (width 0.2) (layer "F.Cu") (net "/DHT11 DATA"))
 (segment (start 185.3295 70.92525) (end 187.0045 72.60025) (width 0.2) (layer "F.Cu") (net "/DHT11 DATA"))
 (segment (start 172 55.04) (end 168 51.04) (width 0.2) (layer "F.Cu") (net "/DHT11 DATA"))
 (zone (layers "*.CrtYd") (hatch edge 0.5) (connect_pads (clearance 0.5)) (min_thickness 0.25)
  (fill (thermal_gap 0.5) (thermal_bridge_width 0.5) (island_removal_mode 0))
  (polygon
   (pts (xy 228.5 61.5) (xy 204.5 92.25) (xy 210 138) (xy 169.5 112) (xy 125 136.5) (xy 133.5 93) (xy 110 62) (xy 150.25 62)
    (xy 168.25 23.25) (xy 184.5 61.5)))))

